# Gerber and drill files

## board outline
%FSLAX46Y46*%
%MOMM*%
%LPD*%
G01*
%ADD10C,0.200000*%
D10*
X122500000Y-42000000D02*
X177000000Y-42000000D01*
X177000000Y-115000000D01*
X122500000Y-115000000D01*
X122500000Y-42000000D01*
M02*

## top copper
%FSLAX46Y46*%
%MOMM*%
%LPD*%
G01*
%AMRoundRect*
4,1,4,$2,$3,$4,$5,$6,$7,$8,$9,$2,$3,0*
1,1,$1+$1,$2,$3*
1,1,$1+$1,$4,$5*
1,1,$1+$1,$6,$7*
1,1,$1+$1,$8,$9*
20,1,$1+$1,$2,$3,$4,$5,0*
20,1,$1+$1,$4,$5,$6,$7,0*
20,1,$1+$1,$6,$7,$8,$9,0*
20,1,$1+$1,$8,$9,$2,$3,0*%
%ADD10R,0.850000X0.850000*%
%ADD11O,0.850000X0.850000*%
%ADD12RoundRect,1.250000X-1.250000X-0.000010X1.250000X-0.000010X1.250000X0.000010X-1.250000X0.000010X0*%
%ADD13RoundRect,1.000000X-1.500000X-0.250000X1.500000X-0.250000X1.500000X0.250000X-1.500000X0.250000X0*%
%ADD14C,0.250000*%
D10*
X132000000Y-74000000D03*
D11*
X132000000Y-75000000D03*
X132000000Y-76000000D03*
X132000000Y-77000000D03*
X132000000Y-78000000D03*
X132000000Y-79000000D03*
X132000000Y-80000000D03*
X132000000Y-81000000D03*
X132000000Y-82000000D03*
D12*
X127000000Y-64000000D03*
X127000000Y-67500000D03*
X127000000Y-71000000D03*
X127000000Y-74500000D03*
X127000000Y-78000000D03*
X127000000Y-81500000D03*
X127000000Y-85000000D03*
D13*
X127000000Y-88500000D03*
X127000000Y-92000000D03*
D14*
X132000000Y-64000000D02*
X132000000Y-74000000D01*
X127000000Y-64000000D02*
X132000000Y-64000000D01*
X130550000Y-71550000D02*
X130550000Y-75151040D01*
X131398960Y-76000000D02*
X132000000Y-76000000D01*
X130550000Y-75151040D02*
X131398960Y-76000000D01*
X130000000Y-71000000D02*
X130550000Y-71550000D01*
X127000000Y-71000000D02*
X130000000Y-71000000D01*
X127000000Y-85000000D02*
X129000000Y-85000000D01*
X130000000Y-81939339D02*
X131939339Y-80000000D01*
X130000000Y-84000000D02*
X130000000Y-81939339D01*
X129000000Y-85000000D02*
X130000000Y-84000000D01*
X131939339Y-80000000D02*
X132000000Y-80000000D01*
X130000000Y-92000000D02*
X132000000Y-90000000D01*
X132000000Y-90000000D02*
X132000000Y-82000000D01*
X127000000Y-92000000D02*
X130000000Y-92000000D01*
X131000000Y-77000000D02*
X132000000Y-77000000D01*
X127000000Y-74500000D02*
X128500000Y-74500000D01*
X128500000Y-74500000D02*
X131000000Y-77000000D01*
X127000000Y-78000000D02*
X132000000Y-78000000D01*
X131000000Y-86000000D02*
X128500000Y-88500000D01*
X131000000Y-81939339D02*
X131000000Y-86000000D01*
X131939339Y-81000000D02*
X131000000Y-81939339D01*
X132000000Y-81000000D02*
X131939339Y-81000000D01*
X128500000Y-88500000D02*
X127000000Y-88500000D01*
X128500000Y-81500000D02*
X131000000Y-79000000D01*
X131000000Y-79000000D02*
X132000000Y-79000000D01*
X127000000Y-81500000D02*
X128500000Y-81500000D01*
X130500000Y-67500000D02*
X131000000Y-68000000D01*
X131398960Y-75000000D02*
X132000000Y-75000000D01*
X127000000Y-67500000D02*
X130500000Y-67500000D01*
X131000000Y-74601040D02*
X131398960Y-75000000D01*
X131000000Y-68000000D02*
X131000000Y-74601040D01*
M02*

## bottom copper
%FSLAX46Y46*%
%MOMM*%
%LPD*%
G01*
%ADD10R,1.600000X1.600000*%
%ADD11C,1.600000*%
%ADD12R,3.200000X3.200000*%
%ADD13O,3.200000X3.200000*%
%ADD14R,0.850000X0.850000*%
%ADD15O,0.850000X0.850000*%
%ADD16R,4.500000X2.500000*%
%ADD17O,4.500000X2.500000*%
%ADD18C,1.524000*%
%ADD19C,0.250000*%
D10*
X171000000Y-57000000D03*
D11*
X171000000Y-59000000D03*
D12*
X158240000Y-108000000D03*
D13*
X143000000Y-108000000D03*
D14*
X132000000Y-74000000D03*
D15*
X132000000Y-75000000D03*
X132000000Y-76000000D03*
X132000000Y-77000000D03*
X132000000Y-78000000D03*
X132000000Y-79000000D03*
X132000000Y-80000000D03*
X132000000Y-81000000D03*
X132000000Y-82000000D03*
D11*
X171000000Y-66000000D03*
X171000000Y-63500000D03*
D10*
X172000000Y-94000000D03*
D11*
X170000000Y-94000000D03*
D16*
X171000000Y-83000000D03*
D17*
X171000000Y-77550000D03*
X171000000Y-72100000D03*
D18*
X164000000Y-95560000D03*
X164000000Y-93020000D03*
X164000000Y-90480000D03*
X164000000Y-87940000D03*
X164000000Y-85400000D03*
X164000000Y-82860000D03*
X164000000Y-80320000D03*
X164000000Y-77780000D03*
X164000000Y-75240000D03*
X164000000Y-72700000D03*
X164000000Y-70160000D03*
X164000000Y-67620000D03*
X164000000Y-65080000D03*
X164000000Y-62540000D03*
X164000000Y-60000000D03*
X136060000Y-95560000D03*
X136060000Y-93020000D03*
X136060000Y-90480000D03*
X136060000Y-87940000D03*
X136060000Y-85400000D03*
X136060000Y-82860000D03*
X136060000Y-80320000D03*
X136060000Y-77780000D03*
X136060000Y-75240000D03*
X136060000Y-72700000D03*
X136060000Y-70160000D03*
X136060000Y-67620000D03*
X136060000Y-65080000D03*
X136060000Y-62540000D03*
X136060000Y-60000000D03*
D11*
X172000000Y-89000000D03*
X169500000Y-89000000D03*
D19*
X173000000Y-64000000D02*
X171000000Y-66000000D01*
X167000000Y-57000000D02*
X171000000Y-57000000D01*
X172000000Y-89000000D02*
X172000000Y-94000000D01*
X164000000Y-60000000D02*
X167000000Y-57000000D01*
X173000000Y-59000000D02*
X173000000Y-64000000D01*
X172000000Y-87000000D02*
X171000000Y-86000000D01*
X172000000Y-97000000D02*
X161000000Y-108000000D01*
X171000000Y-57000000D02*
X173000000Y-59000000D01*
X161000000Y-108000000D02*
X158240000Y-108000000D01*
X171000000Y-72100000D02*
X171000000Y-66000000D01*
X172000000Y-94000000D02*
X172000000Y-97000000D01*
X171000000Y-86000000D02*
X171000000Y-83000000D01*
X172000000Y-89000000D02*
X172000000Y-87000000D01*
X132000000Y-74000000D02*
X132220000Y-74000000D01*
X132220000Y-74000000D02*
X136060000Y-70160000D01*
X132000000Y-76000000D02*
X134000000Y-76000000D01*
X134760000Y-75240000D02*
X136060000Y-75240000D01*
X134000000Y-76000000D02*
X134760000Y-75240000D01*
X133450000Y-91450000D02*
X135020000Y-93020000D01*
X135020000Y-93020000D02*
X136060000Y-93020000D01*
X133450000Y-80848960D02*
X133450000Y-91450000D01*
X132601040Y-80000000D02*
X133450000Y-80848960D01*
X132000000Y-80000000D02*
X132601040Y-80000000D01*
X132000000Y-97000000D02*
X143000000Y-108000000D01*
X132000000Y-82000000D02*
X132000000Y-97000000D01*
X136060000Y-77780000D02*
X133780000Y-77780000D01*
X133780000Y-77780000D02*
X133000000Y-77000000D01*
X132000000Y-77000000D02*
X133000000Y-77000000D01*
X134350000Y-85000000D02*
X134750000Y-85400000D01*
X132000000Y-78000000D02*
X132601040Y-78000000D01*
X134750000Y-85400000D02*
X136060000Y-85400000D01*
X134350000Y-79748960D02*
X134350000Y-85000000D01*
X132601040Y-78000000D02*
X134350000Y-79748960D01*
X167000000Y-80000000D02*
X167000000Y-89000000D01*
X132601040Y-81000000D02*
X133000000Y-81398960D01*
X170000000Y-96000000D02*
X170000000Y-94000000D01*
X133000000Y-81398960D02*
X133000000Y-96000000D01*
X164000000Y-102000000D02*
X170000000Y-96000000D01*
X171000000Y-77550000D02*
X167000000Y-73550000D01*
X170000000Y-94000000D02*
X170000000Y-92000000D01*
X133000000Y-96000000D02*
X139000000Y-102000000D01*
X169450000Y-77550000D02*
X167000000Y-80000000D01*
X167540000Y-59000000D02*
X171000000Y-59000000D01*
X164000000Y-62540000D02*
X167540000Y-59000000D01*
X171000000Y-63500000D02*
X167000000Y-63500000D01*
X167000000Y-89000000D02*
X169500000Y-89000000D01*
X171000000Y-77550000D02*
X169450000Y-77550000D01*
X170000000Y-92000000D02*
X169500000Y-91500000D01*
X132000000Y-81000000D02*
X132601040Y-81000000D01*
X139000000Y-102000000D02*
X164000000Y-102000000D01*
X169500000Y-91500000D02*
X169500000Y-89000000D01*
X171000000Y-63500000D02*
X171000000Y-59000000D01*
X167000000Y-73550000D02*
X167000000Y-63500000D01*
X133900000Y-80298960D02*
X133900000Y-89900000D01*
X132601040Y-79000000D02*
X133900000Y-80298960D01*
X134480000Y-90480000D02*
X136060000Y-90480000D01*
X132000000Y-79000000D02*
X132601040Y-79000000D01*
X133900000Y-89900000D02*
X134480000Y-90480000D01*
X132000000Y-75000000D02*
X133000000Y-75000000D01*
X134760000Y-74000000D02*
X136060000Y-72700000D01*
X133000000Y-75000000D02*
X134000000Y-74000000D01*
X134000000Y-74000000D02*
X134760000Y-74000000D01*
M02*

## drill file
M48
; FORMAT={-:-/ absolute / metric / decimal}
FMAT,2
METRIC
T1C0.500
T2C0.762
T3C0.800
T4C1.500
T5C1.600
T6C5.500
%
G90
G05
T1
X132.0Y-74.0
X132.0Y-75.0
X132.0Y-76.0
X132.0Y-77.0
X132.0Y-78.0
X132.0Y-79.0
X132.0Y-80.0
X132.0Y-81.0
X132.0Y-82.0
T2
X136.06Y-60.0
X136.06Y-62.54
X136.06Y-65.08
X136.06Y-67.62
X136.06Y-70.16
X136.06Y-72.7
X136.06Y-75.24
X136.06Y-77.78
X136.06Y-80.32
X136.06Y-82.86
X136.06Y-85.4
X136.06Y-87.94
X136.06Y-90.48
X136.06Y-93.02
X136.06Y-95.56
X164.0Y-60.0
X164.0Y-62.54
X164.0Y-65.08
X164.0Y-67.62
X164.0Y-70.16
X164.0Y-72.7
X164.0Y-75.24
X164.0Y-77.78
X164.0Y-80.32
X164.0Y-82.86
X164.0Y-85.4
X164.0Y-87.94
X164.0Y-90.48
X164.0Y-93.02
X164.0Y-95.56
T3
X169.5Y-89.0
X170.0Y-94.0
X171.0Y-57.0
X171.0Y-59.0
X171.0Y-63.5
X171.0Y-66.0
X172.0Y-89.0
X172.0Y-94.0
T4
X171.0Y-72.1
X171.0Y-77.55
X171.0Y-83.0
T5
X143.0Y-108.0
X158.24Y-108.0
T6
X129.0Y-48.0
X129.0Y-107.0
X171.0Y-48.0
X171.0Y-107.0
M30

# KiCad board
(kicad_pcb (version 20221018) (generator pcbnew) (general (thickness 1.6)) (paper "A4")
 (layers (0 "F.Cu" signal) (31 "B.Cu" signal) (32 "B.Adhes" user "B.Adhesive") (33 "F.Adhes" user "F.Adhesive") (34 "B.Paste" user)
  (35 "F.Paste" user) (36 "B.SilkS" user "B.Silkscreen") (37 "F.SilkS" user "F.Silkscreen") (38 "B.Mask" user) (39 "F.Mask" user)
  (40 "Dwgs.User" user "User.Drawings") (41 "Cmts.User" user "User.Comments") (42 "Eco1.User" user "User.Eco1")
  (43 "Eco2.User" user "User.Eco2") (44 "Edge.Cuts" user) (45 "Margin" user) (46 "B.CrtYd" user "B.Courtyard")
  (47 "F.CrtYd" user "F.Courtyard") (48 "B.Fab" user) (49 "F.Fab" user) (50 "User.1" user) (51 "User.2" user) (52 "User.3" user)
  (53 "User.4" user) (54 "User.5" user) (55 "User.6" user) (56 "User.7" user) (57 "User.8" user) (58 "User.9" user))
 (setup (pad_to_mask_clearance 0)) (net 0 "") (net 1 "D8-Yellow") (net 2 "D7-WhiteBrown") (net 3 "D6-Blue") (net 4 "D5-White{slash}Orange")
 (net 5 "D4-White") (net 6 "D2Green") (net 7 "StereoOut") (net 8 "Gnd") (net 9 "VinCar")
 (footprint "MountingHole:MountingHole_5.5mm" (layer "F.Cu") (at 129 48)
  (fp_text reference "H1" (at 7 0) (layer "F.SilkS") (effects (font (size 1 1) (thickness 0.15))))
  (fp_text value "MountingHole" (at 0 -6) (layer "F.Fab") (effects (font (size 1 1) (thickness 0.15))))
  (pad "" np_thru_hole circle (at 0 0) (size 5.5 5.5) (drill 5.5) (layers "B.Cu" "B.Mask")))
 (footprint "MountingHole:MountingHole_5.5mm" (layer "F.Cu") (at 171 107)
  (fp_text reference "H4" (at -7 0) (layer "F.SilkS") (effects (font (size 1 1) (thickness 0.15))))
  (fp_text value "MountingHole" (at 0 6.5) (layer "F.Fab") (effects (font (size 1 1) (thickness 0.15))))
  (pad "" np_thru_hole circle (at 0 0) (size 5.5 5.5) (drill 5.5) (layers "B.Cu" "B.Mask")))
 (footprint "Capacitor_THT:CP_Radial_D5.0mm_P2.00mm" (layer "F.Cu") (at 171 57 -90)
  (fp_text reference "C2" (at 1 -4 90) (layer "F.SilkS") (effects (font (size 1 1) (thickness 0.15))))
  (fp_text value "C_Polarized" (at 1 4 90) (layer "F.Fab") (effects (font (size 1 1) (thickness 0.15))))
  (pad "" np_thru_hole rect (at 0 0 270) (size 1.6 1.6) (drill 0.8) (layers "B.Cu" "B.Mask"))
  (pad "" np_thru_hole circle (at 2 0 270) (size 1.6 1.6) (drill 0.8) (layers "B.Cu" "B.Mask")))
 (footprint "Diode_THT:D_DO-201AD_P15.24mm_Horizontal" (layer "F.Cu") (at 158.24 108 180)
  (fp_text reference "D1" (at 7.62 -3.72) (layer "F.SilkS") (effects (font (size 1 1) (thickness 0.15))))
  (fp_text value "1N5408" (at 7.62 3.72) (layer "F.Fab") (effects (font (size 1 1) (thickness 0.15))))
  (pad "" np_thru_hole rect (at 0 0 180) (size 3.2 3.2) (drill 1.6) (layers "B.Cu" "B.Mask"))
  (pad "" np_thru_hole oval (at 15.24 0 180) (size 3.2 3.2) (drill 1.6) (layers "B.Cu" "B.Mask")))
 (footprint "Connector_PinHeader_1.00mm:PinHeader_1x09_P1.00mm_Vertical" (layer "F.Cu") (at 132 74)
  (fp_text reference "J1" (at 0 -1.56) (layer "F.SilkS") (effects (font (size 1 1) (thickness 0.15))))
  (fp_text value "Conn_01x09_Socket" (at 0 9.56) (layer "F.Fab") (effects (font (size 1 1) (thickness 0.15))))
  (pad "1" thru_hole rect (at 0 0) (size 0.85 0.85) (drill 0.5) (layers "*.Cu" "*.Mask") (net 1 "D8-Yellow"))
  (pad "2" thru_hole oval (at 0 1) (size 0.85 0.85) (drill 0.5) (layers "*.Cu" "*.Mask") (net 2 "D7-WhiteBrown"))
  (pad "3" thru_hole oval (at 0 2) (size 0.85 0.85) (drill 0.5) (layers "*.Cu" "*.Mask") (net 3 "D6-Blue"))
  (pad "4" thru_hole oval (at 0 3) (size 0.85 0.85) (drill 0.5) (layers "*.Cu" "*.Mask") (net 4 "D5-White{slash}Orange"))
  (pad "5" thru_hole oval (at 0 4) (size 0.85 0.85) (drill 0.5) (layers "*.Cu" "*.Mask") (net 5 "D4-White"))
  (pad "6" thru_hole oval (at 0 5) (size 0.85 0.85) (drill 0.5) (layers "*.Cu" "*.Mask") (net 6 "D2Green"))
  (pad "7" thru_hole oval (at 0 6) (size 0.85 0.85) (drill 0.5) (layers "*.Cu" "*.Mask") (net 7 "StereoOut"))
  (pad "8" thru_hole oval (at 0 7) (size 0.85 0.85) (drill 0.5) (layers "*.Cu" "*.Mask") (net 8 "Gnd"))
  (pad "9" thru_hole oval (at 0 8) (size 0.85 0.85) (drill 0.5) (layers "*.Cu" "*.Mask") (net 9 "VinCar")))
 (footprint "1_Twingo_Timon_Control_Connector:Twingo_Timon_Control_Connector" (layer "F.Cu") (at 127 78)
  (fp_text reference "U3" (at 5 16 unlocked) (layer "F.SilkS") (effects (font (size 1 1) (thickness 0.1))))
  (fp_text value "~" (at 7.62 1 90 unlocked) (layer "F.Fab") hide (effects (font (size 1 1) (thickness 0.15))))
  (pad "1" smd roundrect (at 0 -14) (size 5 2.5) (layers "F.Cu" "F.Paste" "F.Mask") (roundrect_rratio 0.5) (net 1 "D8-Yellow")
   (thermal_bridge_angle 45))
  (pad "2" smd roundrect (at 0 -10.5) (size 5 2.5) (layers "F.Cu" "F.Paste" "F.Mask") (roundrect_rratio 0.5) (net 2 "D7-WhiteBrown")
   (thermal_bridge_angle 45))
  (pad "3" smd roundrect (at 0 -7) (size 5 2.5) (layers "F.Cu" "F.Paste" "F.Mask") (roundrect_rratio 0.5) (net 3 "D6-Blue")
   (thermal_bridge_angle 45))
  (pad "4" smd roundrect (at 0 -3.5) (size 5 2.5) (layers "F.Cu" "F.Paste" "F.Mask") (roundrect_rratio 0.5) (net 4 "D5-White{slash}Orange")
   (thermal_bridge_angle 45))
  (pad "5" smd roundrect (at 0 0) (size 5 2.5) (layers "F.Cu" "F.Paste" "F.Mask") (roundrect_rratio 0.5) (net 5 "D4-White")
   (thermal_bridge_angle 45))
  (pad "6" smd roundrect (at 0 3.5) (size 5 2.5) (layers "F.Cu" "F.Paste" "F.Mask") (roundrect_rratio 0.5) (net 6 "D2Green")
   (thermal_bridge_angle 45))
  (pad "7" smd roundrect (at 0 7) (size 5 2.5) (layers "F.Cu" "F.Paste" "F.Mask") (roundrect_rratio 0.5) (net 7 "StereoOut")
   (thermal_bridge_angle 45))
  (pad "8" smd roundrect (at 0 10.5) (size 5 2.5) (layers "F.Cu" "F.Paste" "F.Mask") (roundrect_rratio 0.4) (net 8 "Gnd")
   (thermal_bridge_angle 45))
  (pad "9" smd roundrect (at 0 14) (size 5 2.5) (layers "F.Cu" "F.Paste" "F.Mask") (roundrect_rratio 0.4) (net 9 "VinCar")
   (thermal_bridge_angle 45)))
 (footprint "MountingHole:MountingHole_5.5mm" (layer "F.Cu") (at 171 48)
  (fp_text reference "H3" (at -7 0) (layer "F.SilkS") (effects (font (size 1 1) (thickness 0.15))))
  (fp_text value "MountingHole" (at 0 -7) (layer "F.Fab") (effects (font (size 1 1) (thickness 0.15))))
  (pad "" np_thru_hole circle (at 0 0) (size 5.5 5.5) (drill 5.5) (layers "B.Cu" "B.Mask")))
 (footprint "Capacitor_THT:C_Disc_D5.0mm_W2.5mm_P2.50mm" (layer "F.Cu") (at 171 66 90)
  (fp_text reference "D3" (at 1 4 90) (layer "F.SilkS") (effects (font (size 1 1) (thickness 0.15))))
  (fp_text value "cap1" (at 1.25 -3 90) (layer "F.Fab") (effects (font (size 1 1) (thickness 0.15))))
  (pad "" np_thru_hole circle (at 0 0 90) (size 1.6 1.6) (drill 0.8) (layers "B.Cu" "B.Mask"))
  (pad "" np_thru_hole circle (at 2.5 0 90) (size 1.6 1.6) (drill 0.8) (layers "B.Cu" "B.Mask")))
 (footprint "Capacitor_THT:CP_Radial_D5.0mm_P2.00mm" (layer "F.Cu") (at 172 94 180)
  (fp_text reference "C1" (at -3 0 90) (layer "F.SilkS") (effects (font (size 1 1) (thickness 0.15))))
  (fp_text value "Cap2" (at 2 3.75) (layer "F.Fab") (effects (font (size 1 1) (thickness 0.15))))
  (pad "" np_thru_hole rect (at 0 0 180) (size 1.6 1.6) (drill 0.8) (layers "B.Cu" "B.Mask"))
  (pad "" np_thru_hole circle (at 2 0 180) (size 1.6 1.6) (drill 0.8) (layers "B.Cu" "B.Mask")))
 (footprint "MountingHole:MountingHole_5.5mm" (layer "F.Cu") (at 129 107)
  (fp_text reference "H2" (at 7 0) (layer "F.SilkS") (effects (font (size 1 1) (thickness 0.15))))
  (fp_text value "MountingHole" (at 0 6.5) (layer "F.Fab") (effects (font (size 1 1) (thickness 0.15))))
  (pad "" np_thru_hole circle (at 0 0) (size 5.5 5.5) (drill 5.5) (layers "B.Cu" "B.Mask")))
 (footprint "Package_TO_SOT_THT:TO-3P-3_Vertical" (layer "F.Cu") (at 171 83 90)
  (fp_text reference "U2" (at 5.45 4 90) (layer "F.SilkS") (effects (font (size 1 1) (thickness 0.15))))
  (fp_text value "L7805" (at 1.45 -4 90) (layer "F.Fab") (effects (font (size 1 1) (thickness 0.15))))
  (pad "" np_thru_hole rect (at 0 0 90) (size 2.5 4.5) (drill 1.5) (layers "B.Cu" "B.Mask"))
  (pad "" np_thru_hole oval (at 5.45 0 90) (size 2.5 4.5) (drill 1.5) (layers "B.Cu" "B.Mask"))
  (pad "" np_thru_hole oval (at 10.9 0 90) (size 2.5 4.5) (drill 1.5) (layers "B.Cu" "B.Mask")))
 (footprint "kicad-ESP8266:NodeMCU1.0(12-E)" (layer "F.Cu") (at 150.03 77.78 180)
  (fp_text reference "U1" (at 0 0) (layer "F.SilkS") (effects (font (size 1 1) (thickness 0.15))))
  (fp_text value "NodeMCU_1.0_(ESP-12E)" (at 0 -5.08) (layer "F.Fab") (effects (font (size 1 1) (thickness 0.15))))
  (pad "" np_thru_hole circle (at -13.97 -17.78 180) (size 1.524 1.524) (drill 0.762) (layers "B.Cu" "B.Mask"))
  (pad "" np_thru_hole circle (at -13.97 -15.24 180) (size 1.524 1.524) (drill 0.762) (layers "B.Cu" "B.Mask"))
  (pad "" np_thru_hole circle (at -13.97 -12.7 180) (size 1.524 1.524) (drill 0.762) (layers "B.Cu" "B.Mask"))
  (pad "" np_thru_hole circle (at -13.97 -10.16 180) (size 1.524 1.524) (drill 0.762) (layers "B.Cu" "B.Mask"))
  (pad "" np_thru_hole circle (at -13.97 -7.62 180) (size 1.524 1.524) (drill 0.762) (layers "B.Cu" "B.Mask"))
  (pad "" np_thru_hole circle (at -13.97 -5.08 180) (size 1.524 1.524) (drill 0.762) (layers "B.Cu" "B.Mask"))
  (pad "" np_thru_hole circle (at -13.97 -2.54 180) (size 1.524 1.524) (drill 0.762) (layers "B.Cu" "B.Mask"))
  (pad "" np_thru_hole circle (at -13.97 0 180) (size 1.524 1.524) (drill 0.762) (layers "B.Cu" "B.Mask"))
  (pad "" np_thru_hole circle (at -13.97 2.54 180) (size 1.524 1.524) (drill 0.762) (layers "B.Cu" "B.Mask"))
  (pad "" np_thru_hole circle (at -13.97 5.08 180) (size 1.524 1.524) (drill 0.762) (layers "B.Cu" "B.Mask"))
  (pad "" np_thru_hole circle (at -13.97 7.62 180) (size 1.524 1.524) (drill 0.762) (layers "B.Cu" "B.Mask"))
  (pad "" np_thru_hole circle (at -13.97 10.16 180) (size 1.524 1.524) (drill 0.762) (layers "B.Cu" "B.Mask"))
  (pad "" np_thru_hole circle (at -13.97 12.7 180) (size 1.524 1.524) (drill 0.762) (layers "B.Cu" "B.Mask"))
  (pad "" np_thru_hole circle (at -13.97 15.24 180) (size 1.524 1.524) (drill 0.762) (layers "B.Cu" "B.Mask"))
  (pad "" np_thru_hole circle (at -13.97 17.78 180) (size 1.524 1.524) (drill 0.762) (layers "B.Cu" "B.Mask"))
  (pad "" np_thru_hole circle (at 13.97 -17.78 180) (size 1.524 1.524) (drill 0.762) (layers "B.Cu" "B.Mask"))
  (pad "" np_thru_hole circle (at 13.97 -15.24 180) (size 1.524 1.524) (drill 0.762) (layers "B.Cu" "B.Mask"))
  (pad "" np_thru_hole circle (at 13.97 -12.7 180) (size 1.524 1.524) (drill 0.762) (layers "B.Cu" "B.Mask"))
  (pad "" np_thru_hole circle (at 13.97 -10.16 180) (size 1.524 1.524) (drill 0.762) (layers "B.Cu" "B.Mask"))
  (pad "" np_thru_hole circle (at 13.97 -7.62 180) (size 1.524 1.524) (drill 0.762) (layers "B.Cu" "B.Mask"))
  (pad "" np_thru_hole circle (at 13.97 -5.08 180) (size 1.524 1.524) (drill 0.762) (layers "B.Cu" "B.Mask"))
  (pad "" np_thru_hole circle (at 13.97 -2.54 180) (size 1.524 1.524) (drill 0.762) (layers "B.Cu" "B.Mask"))
  (pad "" np_thru_hole circle (at 13.97 0 180) (size 1.524 1.524) (drill 0.762) (layers "B.Cu" "B.Mask"))
  (pad "" np_thru_hole circle (at 13.97 2.54 180) (size 1.524 1.524) (drill 0.762) (layers "B.Cu" "B.Mask"))
  (pad "" np_thru_hole circle (at 13.97 5.08 180) (size 1.524 1.524) (drill 0.762) (layers "B.Cu" "B.Mask"))
  (pad "" np_thru_hole circle (at 13.97 7.62 180) (size 1.524 1.524) (drill 0.762) (layers "B.Cu" "B.Mask"))
  (pad "" np_thru_hole circle (at 13.97 10.16 180) (size 1.524 1.524) (drill 0.762) (layers "B.Cu" "B.Mask"))
  (pad "" np_thru_hole circle (at 13.97 12.7 180) (size 1.524 1.524) (drill 0.762) (layers "B.Cu" "B.Mask"))
  (pad "" np_thru_hole circle (at 13.97 15.24 180) (size 1.524 1.524) (drill 0.762) (layers "B.Cu" "B.Mask"))
  (pad "" np_thru_hole circle (at 13.97 17.78 180) (size 1.524 1.524) (drill 0.762) (layers "B.Cu" "B.Mask")))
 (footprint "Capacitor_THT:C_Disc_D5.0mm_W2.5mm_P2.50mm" (layer "F.Cu") (at 172 89 180)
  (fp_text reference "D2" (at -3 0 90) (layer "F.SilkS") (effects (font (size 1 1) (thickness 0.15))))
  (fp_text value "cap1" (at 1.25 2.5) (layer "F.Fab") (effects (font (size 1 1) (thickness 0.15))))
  (pad "" np_thru_hole circle (at 0 0 180) (size 1.6 1.6) (drill 0.8) (layers "B.Cu" "B.Mask"))
  (pad "" np_thru_hole circle (at 2.5 0 180) (size 1.6 1.6) (drill 0.8) (layers "B.Cu" "B.Mask")))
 (gr_rect (start 122.5 42) (end 177 115) (stroke (width 0.2) (type default)) (fill none) (layer "Edge.Cuts"))
 (segment (start 173 64) (end 171 66) (width 0.25) (layer "B.Cu") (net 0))
 (segment (start 167 57) (end 171 57) (width 0.25) (layer "B.Cu") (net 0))
 (segment (start 172 89) (end 172 94) (width 0.25) (layer "B.Cu") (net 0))
 (segment (start 164 60) (end 167 57) (width 0.25) (layer "B.Cu") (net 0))
 (segment (start 173 59) (end 173 64) (width 0.25) (layer "B.Cu") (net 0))
 (segment (start 172 87) (end 171 86) (width 0.25) (layer "B.Cu") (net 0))
 (segment (start 172 97) (end 161 108) (width 0.25) (layer "B.Cu") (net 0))
 (segment (start 171 57) (end 173 59) (width 0.25) (layer "B.Cu") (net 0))
 (segment (start 161 108) (end 158.24 108) (width 0.25) (layer "B.Cu") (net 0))
 (segment (start 171 72.1) (end 171 66) (width 0.25) (layer "B.Cu") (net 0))
 (segment (start 172 94) (end 172 97) (width 0.25) (layer "B.Cu") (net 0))
 (segment (start 171 86) (end 171 83) (width 0.25) (layer "B.Cu") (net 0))
 (segment (start 172 89) (end 172 87) (width 0.25) (layer "B.Cu") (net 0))
 (segment (start 132 64) (end 132 74) (width 0.25) (layer "F.Cu") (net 1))
 (segment (start 127 64) (end 132 64) (width 0.25) (layer "F.Cu") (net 1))
 (segment (start 132 74) (end 132.22 74) (width 0.25) (layer "B.Cu") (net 1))
 (segment (start 132.22 74) (end 136.06 70.16) (width 0.25) (layer "B.Cu") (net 1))
 (segment (start 130.55 71.55) (end 130.55 75.15104) (width 0.25) (layer "F.Cu") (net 3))
 (segment (start 131.39896 76) (end 132 76) (width 0.25) (layer "F.Cu") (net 3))
 (segment (start 130.55 75.15104) (end 131.39896 76) (width 0.25) (layer "F.Cu") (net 3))
 (segment (start 130 71) (end 130.55 71.55) (width 0.25) (layer "F.Cu") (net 3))
 (segment (start 127 71) (end 130 71) (width 0.25) (layer "F.Cu") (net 3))
 (segment (start 132 76) (end 134 76) (width 0.25) (layer "B.Cu") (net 3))
 (segment (start 134.76 75.24) (end 136.06 75.24) (width 0.25) (layer "B.Cu") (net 3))
 (segment (start 134 76) (end 134.76 75.24) (width 0.25) (layer "B.Cu") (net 3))
 (segment (start 127 85) (end 129 85) (width 0.25) (layer "F.Cu") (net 7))
 (segment (start 130 81.939339) (end 131.939339 80) (width 0.25) (layer "F.Cu") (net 7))
 (segment (start 130 84) (end 130 81.939339) (width 0.25) (layer "F.Cu") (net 7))
 (segment (start 129 85) (end 130 84) (width 0.25) (layer "F.Cu") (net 7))
 (segment (start 131.939339 80) (end 132 80) (width 0.25) (layer "F.Cu") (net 7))
 (segment (start 133.45 91.45) (end 135.02 93.02) (width 0.25) (layer "B.Cu") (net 7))
 (segment (start 135.02 93.02) (end 136.06 93.02) (width 0.25) (layer "B.Cu") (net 7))
 (segment (start 133.45 80.84896) (end 133.45 91.45) (width 0.25) (layer "B.Cu") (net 7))
 (segment (start 132.60104 80) (end 133.45 80.84896) (width 0.25) (layer "B.Cu") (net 7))
 (segment (start 132 80) (end 132.60104 80) (width 0.25) (layer "B.Cu") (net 7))
 (segment (start 130 92) (end 132 90) (width 0.25) (layer "F.Cu") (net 9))
 (segment (start 132 90) (end 132 82) (width 0.25) (layer "F.Cu") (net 9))
 (segment (start 127 92) (end 130 92) (width 0.25) (layer "F.Cu") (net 9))
 (segment (start 132 97) (end 143 108) (width 0.25) (layer "B.Cu") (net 9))
 (segment (start 132 82) (end 132 97) (width 0.25) (layer "B.Cu") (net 9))
 (segment (start 131 77) (end 132 77) (width 0.25) (layer "F.Cu") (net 4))
 (segment (start 127 74.5) (end 128.5 74.5) (width 0.25) (layer "F.Cu") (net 4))
 (segment (start 128.5 74.5) (end 131 77) (width 0.25) (layer "F.Cu") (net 4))
 (segment (start 136.06 77.78) (end 133.78 77.78) (width 0.25) (layer "B.Cu") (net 4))
 (segment (start 133.78 77.78) (end 133 77) (width 0.25) (layer "B.Cu") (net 4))
 (segment (start 132 77) (end 133 77) (width 0.25) (layer "B.Cu") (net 4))
 (segment (start 127 78) (end 132 78) (width 0.25) (layer "F.Cu") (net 5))
 (segment (start 134.35 85) (end 134.75 85.4) (width 0.25) (layer "B.Cu") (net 5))
 (segment (start 132 78) (end 132.60104 78) (width 0.25) (layer "B.Cu") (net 5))
 (segment (start 134.75 85.4) (end 136.06 85.4) (width 0.25) (layer "B.Cu") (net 5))
 (segment (start 134.35 79.74896) (end 134.35 85) (width 0.25) (layer "B.Cu") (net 5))
 (segment (start 132.60104 78) (end 134.35 79.74896) (width 0.25) (layer "B.Cu") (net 5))
 (segment (start 131 86) (end 128.5 88.5) (width 0.25) (layer "F.Cu") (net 8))
 (segment (start 131 81.939339) (end 131 86) (width 0.25) (layer "F.Cu") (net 8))
 (segment (start 131.939339 81) (end 131 81.939339) (width 0.25) (layer "F.Cu") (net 8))
 (segment (start 132 81) (end 131.939339 81) (width 0.25) (layer "F.Cu") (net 8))
 (segment (start 128.5 88.5) (end 127 88.5) (width 0.25) (layer "F.Cu") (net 8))
 (segment (start 167 80) (end 167 89) (width 0.25) (layer "B.Cu") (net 8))
 (segment (start 132.60104 81) (end 133 81.39896) (width 0.25) (layer "B.Cu") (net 8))
 (segment (start 170 96) (end 170 94) (width 0.25) (layer "B.Cu") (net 8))
 (segment (start 133 81.39896) (end 133 96) (width 0.25) (layer "B.Cu") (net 8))
 (segment (start 164 102) (end 170 96) (width 0.25) (layer "B.Cu") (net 8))
 (segment (start 171 77.55) (end 167 73.55) (width 0.25) (layer "B.Cu") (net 8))
 (segment (start 170 94) (end 170 92) (width 0.25) (layer "B.Cu") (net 8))
 (segment (start 133 96) (end 139 102) (width 0.25) (layer "B.Cu") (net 8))
 (segment (start 169.45 77.55) (end 167 80) (width 0.25) (layer "B.Cu") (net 8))
 (segment (start 167.54 59) (end 171 59) (width 0.25) (layer "B.Cu") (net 8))
 (segment (start 164 62.54) (end 167.54 59) (width 0.25) (layer "B.Cu") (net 8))
 (segment (start 171 63.5) (end 167 63.5) (width 0.25) (layer "B.Cu") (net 8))
 (segment (start 167 89) (end 169.5 89) (width 0.25) (layer "B.Cu") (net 8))
 (segment (start 171 77.55) (end 169.45 77.55) (width 0.25) (layer "B.Cu") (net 8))
 (segment (start 170 92) (end 169.5 91.5) (width 0.25) (layer "B.Cu") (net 8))
 (segment (start 132 81) (end 132.60104 81) (width 0.25) (layer "B.Cu") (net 8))
 (segment (start 139 102) (end 164 102) (width 0.25) (layer "B.Cu") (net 8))
 (segment (start 169.5 91.5) (end 169.5 89) (width 0.25) (layer "B.Cu") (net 8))
 (segment (start 171 63.5) (end 171 59) (width 0.25) (layer "B.Cu") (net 8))
 (segment (start 167 73.55) (end 167 63.5) (width 0.25) (layer "B.Cu") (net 8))
 (segment (start 128.5 81.5) (end 131 79) (width 0.25) (layer "F.Cu") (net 6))
 (segment (start 131 79) (end 132 79) (width 0.25) (layer "F.Cu") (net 6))
 (segment (start 127 81.5) (end 128.5 81.5) (width 0.25) (layer "F.Cu") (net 6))
 (segment (start 133.9 80.29896) (end 133.9 89.9) (width 0.25) (layer "B.Cu") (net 6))
 (segment (start 132.60104 79) (end 133.9 80.29896) (width 0.25) (layer "B.Cu") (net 6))
 (segment (start 134.48 90.48) (end 136.06 90.48) (width 0.25) (layer "B.Cu") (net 6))
 (segment (start 132 79) (end 132.60104 79) (width 0.25) (layer "B.Cu") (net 6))
 (segment (start 133.9 89.9) (end 134.48 90.48) (width 0.25) (layer "B.Cu") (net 6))
 (segment (start 130.5 67.5) (end 131 68) (width 0.25) (layer "F.Cu") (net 2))
 (segment (start 131.39896 75) (end 132 75) (width 0.25) (layer "F.Cu") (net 2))
 (segment (start 127 67.5) (end 130.5 67.5) (width 0.25) (layer "F.Cu") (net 2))
 (segment (start 131 74.60104) (end 131.39896 75) (width 0.25) (layer "F.Cu") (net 2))
 (segment (start 131 68) (end 131 74.60104) (width 0.25) (layer "F.Cu") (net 2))
 (segment (start 132 75) (end 133 75) (width 0.25) (layer "B.Cu") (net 2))
 (segment (start 134.76 74) (end 136.06 72.7) (width 0.25) (layer "B.Cu") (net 2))
 (segment (start 133 75) (end 134 74) (width 0.25) (layer "B.Cu") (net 2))
 (segment (start 134 74) (end 134.76 74) (width 0.25) (layer "B.Cu") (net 2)))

